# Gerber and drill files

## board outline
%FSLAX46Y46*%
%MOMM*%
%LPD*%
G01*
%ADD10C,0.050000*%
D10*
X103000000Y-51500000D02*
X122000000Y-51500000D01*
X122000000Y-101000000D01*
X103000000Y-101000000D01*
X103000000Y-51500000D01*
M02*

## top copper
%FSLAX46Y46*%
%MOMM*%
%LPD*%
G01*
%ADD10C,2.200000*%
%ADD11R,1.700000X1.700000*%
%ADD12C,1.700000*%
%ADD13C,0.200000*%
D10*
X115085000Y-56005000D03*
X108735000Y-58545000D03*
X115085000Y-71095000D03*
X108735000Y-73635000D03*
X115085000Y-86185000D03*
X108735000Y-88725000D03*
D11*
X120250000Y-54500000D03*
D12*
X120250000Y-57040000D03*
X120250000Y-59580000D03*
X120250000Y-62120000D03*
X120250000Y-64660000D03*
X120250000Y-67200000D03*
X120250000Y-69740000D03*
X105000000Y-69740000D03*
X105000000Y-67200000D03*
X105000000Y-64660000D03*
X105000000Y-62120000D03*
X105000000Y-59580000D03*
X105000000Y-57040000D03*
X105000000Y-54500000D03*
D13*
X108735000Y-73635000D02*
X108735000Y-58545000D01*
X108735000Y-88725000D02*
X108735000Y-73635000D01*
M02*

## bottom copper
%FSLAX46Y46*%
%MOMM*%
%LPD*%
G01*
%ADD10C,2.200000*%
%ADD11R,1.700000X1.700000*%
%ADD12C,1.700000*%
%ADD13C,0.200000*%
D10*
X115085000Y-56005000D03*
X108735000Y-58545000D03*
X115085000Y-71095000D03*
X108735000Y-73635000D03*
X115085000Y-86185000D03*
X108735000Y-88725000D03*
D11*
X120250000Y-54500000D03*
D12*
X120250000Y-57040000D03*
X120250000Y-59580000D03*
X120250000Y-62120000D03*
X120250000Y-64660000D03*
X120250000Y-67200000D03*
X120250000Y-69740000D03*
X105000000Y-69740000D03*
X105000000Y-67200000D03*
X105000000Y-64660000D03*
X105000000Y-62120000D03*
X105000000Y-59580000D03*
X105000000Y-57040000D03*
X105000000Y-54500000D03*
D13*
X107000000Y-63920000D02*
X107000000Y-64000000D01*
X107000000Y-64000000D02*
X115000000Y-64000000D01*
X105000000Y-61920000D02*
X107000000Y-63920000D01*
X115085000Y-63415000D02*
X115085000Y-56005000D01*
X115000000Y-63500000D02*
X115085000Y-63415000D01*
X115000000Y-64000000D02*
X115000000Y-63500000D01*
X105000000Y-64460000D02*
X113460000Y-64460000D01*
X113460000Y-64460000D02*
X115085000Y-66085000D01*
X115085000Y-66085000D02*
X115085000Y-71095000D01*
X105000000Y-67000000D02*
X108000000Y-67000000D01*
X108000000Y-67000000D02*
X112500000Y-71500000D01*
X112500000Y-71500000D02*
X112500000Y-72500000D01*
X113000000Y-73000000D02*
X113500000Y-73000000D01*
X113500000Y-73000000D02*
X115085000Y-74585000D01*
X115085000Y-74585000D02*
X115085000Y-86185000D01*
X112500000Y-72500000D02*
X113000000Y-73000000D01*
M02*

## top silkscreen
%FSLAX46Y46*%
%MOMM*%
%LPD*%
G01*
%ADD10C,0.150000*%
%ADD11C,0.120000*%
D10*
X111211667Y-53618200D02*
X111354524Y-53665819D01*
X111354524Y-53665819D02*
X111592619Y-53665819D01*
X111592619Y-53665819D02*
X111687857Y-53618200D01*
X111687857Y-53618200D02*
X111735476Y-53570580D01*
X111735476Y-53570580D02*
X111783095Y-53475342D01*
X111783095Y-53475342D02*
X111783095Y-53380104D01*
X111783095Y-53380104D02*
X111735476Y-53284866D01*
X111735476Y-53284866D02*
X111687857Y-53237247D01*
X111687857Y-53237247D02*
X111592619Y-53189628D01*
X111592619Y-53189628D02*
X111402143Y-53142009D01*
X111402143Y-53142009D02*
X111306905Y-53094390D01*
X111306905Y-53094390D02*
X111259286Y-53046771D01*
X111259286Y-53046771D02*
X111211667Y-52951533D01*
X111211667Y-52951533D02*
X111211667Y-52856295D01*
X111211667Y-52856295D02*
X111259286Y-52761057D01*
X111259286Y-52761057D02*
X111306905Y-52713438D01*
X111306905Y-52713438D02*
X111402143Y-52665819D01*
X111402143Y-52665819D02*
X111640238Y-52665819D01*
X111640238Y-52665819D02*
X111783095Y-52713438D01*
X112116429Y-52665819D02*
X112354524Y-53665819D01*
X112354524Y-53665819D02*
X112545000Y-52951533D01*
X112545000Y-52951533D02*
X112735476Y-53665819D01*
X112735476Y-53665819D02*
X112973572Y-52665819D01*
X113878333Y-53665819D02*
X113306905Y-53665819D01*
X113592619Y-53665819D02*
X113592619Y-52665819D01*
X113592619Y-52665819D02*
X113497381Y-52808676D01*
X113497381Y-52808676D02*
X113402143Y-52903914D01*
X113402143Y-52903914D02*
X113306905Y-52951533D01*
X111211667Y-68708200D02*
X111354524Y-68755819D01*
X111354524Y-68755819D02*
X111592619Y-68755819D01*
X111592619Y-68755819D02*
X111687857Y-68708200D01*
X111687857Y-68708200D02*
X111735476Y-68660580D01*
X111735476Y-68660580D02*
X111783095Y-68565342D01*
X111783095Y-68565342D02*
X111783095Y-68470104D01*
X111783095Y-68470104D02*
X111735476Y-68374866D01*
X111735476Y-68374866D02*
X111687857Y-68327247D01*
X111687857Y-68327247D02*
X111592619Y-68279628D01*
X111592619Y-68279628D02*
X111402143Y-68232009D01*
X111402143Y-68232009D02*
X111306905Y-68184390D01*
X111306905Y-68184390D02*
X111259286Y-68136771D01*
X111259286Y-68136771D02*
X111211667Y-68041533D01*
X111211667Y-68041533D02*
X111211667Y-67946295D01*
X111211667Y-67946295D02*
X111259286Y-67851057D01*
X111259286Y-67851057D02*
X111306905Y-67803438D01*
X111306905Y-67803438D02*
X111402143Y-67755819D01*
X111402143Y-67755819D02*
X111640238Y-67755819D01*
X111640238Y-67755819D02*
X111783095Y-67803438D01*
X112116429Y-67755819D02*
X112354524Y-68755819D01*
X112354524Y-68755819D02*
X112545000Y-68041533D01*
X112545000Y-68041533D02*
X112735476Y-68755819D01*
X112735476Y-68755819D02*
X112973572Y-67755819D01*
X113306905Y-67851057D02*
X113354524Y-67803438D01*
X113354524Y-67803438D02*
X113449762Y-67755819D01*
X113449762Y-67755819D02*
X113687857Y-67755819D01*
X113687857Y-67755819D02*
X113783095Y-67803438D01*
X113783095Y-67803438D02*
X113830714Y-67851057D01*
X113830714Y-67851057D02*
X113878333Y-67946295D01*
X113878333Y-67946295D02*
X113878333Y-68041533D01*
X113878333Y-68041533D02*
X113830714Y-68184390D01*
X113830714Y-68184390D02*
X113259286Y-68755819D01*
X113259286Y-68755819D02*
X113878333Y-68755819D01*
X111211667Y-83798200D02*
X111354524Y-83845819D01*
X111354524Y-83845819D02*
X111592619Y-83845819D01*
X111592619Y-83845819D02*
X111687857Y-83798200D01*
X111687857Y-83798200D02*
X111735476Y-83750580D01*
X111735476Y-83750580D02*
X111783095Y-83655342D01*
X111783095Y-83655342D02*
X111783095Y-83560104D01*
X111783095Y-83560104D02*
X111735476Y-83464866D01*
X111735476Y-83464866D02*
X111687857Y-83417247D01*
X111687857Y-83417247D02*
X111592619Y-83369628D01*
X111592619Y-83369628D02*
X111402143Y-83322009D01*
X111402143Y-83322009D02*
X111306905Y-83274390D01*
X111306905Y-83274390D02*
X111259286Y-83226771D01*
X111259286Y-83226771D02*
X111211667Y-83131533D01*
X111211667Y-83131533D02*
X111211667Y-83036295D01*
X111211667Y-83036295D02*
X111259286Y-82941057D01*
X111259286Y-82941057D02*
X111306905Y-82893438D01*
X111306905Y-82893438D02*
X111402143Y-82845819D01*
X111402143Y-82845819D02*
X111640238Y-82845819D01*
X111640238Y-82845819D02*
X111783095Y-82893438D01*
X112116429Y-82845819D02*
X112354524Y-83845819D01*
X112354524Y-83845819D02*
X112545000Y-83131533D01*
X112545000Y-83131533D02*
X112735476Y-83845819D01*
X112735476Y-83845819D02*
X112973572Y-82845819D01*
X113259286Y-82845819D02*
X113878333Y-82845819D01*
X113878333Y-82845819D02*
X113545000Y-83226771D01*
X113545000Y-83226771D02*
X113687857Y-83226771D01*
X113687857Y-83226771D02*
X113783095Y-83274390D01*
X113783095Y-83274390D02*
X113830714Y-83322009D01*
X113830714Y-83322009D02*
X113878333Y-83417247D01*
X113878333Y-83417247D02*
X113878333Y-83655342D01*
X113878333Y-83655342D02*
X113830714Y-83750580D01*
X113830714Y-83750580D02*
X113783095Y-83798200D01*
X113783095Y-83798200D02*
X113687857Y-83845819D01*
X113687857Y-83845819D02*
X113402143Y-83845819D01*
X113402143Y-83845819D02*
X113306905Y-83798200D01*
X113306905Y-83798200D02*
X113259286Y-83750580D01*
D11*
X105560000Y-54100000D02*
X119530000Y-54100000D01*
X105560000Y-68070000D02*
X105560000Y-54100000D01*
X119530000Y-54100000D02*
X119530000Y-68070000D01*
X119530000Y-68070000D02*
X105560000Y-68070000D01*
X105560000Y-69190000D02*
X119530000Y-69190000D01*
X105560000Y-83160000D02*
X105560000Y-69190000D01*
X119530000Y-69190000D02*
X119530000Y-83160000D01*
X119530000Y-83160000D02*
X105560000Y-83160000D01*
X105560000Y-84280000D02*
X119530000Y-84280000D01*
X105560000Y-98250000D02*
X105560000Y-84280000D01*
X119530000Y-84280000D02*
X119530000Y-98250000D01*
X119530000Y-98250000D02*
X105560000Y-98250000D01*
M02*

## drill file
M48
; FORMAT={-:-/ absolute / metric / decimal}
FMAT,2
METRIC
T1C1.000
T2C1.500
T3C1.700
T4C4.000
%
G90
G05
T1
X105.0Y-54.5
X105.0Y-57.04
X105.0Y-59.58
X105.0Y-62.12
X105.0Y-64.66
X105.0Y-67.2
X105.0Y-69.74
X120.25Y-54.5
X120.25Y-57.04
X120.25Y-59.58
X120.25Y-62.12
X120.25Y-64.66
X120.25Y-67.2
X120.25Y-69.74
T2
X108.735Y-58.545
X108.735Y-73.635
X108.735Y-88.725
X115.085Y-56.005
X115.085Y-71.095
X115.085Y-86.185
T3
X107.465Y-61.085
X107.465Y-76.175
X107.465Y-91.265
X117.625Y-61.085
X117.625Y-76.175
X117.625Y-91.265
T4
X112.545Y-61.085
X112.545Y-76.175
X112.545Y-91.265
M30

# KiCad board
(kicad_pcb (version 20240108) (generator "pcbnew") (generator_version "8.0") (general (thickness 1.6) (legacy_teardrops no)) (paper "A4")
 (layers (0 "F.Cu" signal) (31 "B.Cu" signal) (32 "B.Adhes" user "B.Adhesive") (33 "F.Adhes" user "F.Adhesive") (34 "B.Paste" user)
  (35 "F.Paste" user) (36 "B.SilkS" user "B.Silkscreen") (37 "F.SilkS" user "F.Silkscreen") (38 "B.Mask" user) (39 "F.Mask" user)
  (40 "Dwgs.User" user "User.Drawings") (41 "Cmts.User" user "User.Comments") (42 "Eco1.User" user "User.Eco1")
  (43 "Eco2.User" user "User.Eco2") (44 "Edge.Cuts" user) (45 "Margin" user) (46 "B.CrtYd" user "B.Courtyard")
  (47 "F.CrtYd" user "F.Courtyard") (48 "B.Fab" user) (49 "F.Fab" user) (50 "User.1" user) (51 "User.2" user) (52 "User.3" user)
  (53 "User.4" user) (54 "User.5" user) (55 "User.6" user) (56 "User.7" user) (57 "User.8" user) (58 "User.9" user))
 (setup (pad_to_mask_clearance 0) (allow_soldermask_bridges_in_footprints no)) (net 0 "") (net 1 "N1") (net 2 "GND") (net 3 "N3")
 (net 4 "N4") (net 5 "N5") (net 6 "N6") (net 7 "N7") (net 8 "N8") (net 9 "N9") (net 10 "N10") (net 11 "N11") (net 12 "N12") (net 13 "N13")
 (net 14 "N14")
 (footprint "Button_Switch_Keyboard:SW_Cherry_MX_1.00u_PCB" (layer "F.Cu") (at 115.085 56.005)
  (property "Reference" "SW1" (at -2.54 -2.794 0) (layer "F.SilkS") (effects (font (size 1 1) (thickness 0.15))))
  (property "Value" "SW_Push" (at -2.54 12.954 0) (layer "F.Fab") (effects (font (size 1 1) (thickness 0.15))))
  (fp_line (start -9.525 -1.905) (end 4.445 -1.905) (stroke (width 0.12) (type solid)) (layer "F.SilkS"))
  (fp_line (start -9.525 12.065) (end -9.525 -1.905) (stroke (width 0.12) (type solid)) (layer "F.SilkS"))
  (fp_line (start 4.445 -1.905) (end 4.445 12.065) (stroke (width 0.12) (type solid)) (layer "F.SilkS"))
  (fp_line (start 4.445 12.065) (end -9.525 12.065) (stroke (width 0.12) (type solid)) (layer "F.SilkS"))
  (pad "" np_thru_hole circle (at -7.62 5.08) (size 1.7 1.7) (drill 1.7) (layers "*.Cu" "*.Mask"))
  (pad "" np_thru_hole circle (at -2.54 5.08) (size 4 4) (drill 4) (layers "*.Cu" "*.Mask"))
  (pad "" np_thru_hole circle (at 2.54 5.08) (size 1.7 1.7) (drill 1.7) (layers "*.Cu" "*.Mask"))
  (pad "1" thru_hole circle (at 0 0) (size 2.2 2.2) (drill 1.5) (layers "*.Cu" "*.Mask") (remove_unused_layers no) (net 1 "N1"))
  (pad "2" thru_hole circle (at -6.35 2.54) (size 2.2 2.2) (drill 1.5) (layers "*.Cu" "*.Mask") (remove_unused_layers no) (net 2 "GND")))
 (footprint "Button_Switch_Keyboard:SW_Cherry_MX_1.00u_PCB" (layer "F.Cu") (at 115.085 71.095)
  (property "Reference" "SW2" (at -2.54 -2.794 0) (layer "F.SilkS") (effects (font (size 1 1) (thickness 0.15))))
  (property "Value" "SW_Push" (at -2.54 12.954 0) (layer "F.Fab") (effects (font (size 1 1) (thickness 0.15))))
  (fp_line (start -9.525 -1.905) (end 4.445 -1.905) (stroke (width 0.12) (type solid)) (layer "F.SilkS"))
  (fp_line (start -9.525 12.065) (end -9.525 -1.905) (stroke (width 0.12) (type solid)) (layer "F.SilkS"))
  (fp_line (start 4.445 -1.905) (end 4.445 12.065) (stroke (width 0.12) (type solid)) (layer "F.SilkS"))
  (fp_line (start 4.445 12.065) (end -9.525 12.065) (stroke (width 0.12) (type solid)) (layer "F.SilkS"))
  (pad "" np_thru_hole circle (at -7.62 5.08) (size 1.7 1.7) (drill 1.7) (layers "*.Cu" "*.Mask"))
  (pad "" np_thru_hole circle (at -2.54 5.08) (size 4 4) (drill 4) (layers "*.Cu" "*.Mask"))
  (pad "" np_thru_hole circle (at 2.54 5.08) (size 1.7 1.7) (drill 1.7) (layers "*.Cu" "*.Mask"))
  (pad "1" thru_hole circle (at 0 0) (size 2.2 2.2) (drill 1.5) (layers "*.Cu" "*.Mask") (remove_unused_layers no) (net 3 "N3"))
  (pad "2" thru_hole circle (at -6.35 2.54) (size 2.2 2.2) (drill 1.5) (layers "*.Cu" "*.Mask") (remove_unused_layers no) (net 2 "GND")))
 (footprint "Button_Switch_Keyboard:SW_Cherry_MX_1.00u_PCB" (layer "F.Cu") (at 115.085 86.185)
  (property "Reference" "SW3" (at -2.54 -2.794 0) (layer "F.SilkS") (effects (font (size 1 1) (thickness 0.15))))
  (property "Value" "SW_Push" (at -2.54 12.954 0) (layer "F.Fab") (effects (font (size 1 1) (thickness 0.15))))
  (fp_line (start -9.525 -1.905) (end 4.445 -1.905) (stroke (width 0.12) (type solid)) (layer "F.SilkS"))
  (fp_line (start -9.525 12.065) (end -9.525 -1.905) (stroke (width 0.12) (type solid)) (layer "F.SilkS"))
  (fp_line (start 4.445 -1.905) (end 4.445 12.065) (stroke (width 0.12) (type solid)) (layer "F.SilkS"))
  (fp_line (start 4.445 12.065) (end -9.525 12.065) (stroke (width 0.12) (type solid)) (layer "F.SilkS"))
  (pad "" np_thru_hole circle (at -7.62 5.08) (size 1.7 1.7) (drill 1.7) (layers "*.Cu" "*.Mask"))
  (pad "" np_thru_hole circle (at -2.54 5.08) (size 4 4) (drill 4) (layers "*.Cu" "*.Mask"))
  (pad "" np_thru_hole circle (at 2.54 5.08) (size 1.7 1.7) (drill 1.7) (layers "*.Cu" "*.Mask"))
  (pad "1" thru_hole circle (at 0 0) (size 2.2 2.2) (drill 1.5) (layers "*.Cu" "*.Mask") (remove_unused_layers no) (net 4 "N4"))
  (pad "2" thru_hole circle (at -6.35 2.54) (size 2.2 2.2) (drill 1.5) (layers "*.Cu" "*.Mask") (remove_unused_layers no) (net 2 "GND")))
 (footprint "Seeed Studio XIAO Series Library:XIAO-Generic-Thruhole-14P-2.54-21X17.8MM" (layer "B.Cu") (at 112.625 62.12 180)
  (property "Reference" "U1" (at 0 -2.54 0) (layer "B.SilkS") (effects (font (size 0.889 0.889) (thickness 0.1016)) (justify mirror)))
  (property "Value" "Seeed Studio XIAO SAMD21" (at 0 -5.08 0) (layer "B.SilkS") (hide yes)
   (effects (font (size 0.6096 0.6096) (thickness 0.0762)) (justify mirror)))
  (pad "1" thru_hole rect (at -7.625 7.62 180) (size 1.7 1.7) (drill 1) (layers "*.Cu" "*.Mask") (remove_unused_layers no) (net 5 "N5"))
  (pad "2" thru_hole circle (at -7.625 5.08 180) (size 1.7 1.7) (drill 1) (layers "*.Cu" "*.Mask") (remove_unused_layers no) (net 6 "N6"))
  (pad "3" thru_hole circle (at -7.625 2.54 180) (size 1.7 1.7) (drill 1) (layers "*.Cu" "*.Mask") (remove_unused_layers no) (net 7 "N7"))
  (pad "4" thru_hole circle (at -7.625 0 180) (size 1.7 1.7) (drill 1) (layers "*.Cu" "*.Mask") (remove_unused_layers no) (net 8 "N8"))
  (pad "5" thru_hole circle (at -7.625 -2.54 180) (size 1.7 1.7) (drill 1) (layers "*.Cu" "*.Mask") (remove_unused_layers no) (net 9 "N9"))
  (pad "6" thru_hole circle (at -7.625 -5.08) (size 1.7 1.7) (drill 1) (layers "*.Cu" "*.Mask") (remove_unused_layers no) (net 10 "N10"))
  (pad "7" thru_hole circle (at -7.625 -7.62 180) (size 1.7 1.7) (drill 1) (layers "*.Cu" "*.Mask") (remove_unused_layers no) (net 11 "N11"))
  (pad "8" thru_hole circle (at 7.625 -7.62 180) (size 1.7 1.7) (drill 1) (layers "*.Cu" "*.Mask") (remove_unused_layers no) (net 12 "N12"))
  (pad "9" thru_hole circle (at 7.625 -5.08 180) (size 1.7 1.7) (drill 1) (layers "*.Cu" "*.Mask") (remove_unused_layers no) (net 4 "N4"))
  (pad "10" thru_hole circle (at 7.625 -2.54 180) (size 1.7 1.7) (drill 1) (layers "*.Cu" "*.Mask") (remove_unused_layers no) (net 3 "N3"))
  (pad "11" thru_hole circle (at 7.625 0 180) (size 1.7 1.7) (drill 1) (layers "*.Cu" "*.Mask") (remove_unused_layers no) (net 1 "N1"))
  (pad "12" thru_hole circle (at 7.625 2.54 180) (size 1.7 1.7) (drill 1) (layers "*.Cu" "*.Mask") (remove_unused_layers no) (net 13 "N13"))
  (pad "13" thru_hole circle (at 7.625 5.08 180) (size 1.7 1.7) (drill 1) (layers "*.Cu" "*.Mask") (remove_unused_layers no) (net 2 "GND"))
  (pad "14" thru_hole circle (at 7.625 7.62 180) (size 1.7 1.7) (drill 1) (layers "*.Cu" "*.Mask") (remove_unused_layers no) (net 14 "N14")))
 (gr_rect (start 103 51.5) (end 122 101) (stroke (width 0.05) (type default)) (fill none) (layer "Edge.Cuts"))
 (segment (start 107 63.92) (end 107 64) (width 0.2) (layer "B.Cu") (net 1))
 (segment (start 107 64) (end 115 64) (width 0.2) (layer "B.Cu") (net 1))
 (segment (start 105 61.92) (end 107 63.92) (width 0.2) (layer "B.Cu") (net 1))
 (segment (start 115.085 63.415) (end 115.085 56.005) (width 0.2) (layer "B.Cu") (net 1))
 (segment (start 115 63.5) (end 115.085 63.415) (width 0.2) (layer "B.Cu") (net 1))
 (segment (start 115 64) (end 115 63.5) (width 0.2) (layer "B.Cu") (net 1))
 (segment (start 108.735 73.635) (end 108.735 58.545) (width 0.2) (layer "F.Cu") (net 2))
 (segment (start 108.735 88.725) (end 108.735 73.635) (width 0.2) (layer "F.Cu") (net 2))
 (segment (start 105 64.46) (end 113.46 64.46) (width 0.2) (layer "B.Cu") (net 3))
 (segment (start 113.46 64.46) (end 115.085 66.085) (width 0.2) (layer "B.Cu") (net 3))
 (segment (start 115.085 66.085) (end 115.085 71.095) (width 0.2) (layer "B.Cu") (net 3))
 (segment (start 105 67) (end 108 67) (width 0.2) (layer "B.Cu") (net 4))
 (segment (start 108 67) (end 112.5 71.5) (width 0.2) (layer "B.Cu") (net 4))
 (segment (start 112.5 71.5) (end 112.5 72.5) (width 0.2) (layer "B.Cu") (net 4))
 (segment (start 113 73) (end 113.5 73) (width 0.2) (layer "B.Cu") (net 4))
 (segment (start 113.5 73) (end 115.085 74.585) (width 0.2) (layer "B.Cu") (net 4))
 (segment (start 115.085 74.585) (end 115.085 86.185) (width 0.2) (layer "B.Cu") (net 4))
 (segment (start 112.5 72.5) (end 113 73) (width 0.2) (layer "B.Cu") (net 4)))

